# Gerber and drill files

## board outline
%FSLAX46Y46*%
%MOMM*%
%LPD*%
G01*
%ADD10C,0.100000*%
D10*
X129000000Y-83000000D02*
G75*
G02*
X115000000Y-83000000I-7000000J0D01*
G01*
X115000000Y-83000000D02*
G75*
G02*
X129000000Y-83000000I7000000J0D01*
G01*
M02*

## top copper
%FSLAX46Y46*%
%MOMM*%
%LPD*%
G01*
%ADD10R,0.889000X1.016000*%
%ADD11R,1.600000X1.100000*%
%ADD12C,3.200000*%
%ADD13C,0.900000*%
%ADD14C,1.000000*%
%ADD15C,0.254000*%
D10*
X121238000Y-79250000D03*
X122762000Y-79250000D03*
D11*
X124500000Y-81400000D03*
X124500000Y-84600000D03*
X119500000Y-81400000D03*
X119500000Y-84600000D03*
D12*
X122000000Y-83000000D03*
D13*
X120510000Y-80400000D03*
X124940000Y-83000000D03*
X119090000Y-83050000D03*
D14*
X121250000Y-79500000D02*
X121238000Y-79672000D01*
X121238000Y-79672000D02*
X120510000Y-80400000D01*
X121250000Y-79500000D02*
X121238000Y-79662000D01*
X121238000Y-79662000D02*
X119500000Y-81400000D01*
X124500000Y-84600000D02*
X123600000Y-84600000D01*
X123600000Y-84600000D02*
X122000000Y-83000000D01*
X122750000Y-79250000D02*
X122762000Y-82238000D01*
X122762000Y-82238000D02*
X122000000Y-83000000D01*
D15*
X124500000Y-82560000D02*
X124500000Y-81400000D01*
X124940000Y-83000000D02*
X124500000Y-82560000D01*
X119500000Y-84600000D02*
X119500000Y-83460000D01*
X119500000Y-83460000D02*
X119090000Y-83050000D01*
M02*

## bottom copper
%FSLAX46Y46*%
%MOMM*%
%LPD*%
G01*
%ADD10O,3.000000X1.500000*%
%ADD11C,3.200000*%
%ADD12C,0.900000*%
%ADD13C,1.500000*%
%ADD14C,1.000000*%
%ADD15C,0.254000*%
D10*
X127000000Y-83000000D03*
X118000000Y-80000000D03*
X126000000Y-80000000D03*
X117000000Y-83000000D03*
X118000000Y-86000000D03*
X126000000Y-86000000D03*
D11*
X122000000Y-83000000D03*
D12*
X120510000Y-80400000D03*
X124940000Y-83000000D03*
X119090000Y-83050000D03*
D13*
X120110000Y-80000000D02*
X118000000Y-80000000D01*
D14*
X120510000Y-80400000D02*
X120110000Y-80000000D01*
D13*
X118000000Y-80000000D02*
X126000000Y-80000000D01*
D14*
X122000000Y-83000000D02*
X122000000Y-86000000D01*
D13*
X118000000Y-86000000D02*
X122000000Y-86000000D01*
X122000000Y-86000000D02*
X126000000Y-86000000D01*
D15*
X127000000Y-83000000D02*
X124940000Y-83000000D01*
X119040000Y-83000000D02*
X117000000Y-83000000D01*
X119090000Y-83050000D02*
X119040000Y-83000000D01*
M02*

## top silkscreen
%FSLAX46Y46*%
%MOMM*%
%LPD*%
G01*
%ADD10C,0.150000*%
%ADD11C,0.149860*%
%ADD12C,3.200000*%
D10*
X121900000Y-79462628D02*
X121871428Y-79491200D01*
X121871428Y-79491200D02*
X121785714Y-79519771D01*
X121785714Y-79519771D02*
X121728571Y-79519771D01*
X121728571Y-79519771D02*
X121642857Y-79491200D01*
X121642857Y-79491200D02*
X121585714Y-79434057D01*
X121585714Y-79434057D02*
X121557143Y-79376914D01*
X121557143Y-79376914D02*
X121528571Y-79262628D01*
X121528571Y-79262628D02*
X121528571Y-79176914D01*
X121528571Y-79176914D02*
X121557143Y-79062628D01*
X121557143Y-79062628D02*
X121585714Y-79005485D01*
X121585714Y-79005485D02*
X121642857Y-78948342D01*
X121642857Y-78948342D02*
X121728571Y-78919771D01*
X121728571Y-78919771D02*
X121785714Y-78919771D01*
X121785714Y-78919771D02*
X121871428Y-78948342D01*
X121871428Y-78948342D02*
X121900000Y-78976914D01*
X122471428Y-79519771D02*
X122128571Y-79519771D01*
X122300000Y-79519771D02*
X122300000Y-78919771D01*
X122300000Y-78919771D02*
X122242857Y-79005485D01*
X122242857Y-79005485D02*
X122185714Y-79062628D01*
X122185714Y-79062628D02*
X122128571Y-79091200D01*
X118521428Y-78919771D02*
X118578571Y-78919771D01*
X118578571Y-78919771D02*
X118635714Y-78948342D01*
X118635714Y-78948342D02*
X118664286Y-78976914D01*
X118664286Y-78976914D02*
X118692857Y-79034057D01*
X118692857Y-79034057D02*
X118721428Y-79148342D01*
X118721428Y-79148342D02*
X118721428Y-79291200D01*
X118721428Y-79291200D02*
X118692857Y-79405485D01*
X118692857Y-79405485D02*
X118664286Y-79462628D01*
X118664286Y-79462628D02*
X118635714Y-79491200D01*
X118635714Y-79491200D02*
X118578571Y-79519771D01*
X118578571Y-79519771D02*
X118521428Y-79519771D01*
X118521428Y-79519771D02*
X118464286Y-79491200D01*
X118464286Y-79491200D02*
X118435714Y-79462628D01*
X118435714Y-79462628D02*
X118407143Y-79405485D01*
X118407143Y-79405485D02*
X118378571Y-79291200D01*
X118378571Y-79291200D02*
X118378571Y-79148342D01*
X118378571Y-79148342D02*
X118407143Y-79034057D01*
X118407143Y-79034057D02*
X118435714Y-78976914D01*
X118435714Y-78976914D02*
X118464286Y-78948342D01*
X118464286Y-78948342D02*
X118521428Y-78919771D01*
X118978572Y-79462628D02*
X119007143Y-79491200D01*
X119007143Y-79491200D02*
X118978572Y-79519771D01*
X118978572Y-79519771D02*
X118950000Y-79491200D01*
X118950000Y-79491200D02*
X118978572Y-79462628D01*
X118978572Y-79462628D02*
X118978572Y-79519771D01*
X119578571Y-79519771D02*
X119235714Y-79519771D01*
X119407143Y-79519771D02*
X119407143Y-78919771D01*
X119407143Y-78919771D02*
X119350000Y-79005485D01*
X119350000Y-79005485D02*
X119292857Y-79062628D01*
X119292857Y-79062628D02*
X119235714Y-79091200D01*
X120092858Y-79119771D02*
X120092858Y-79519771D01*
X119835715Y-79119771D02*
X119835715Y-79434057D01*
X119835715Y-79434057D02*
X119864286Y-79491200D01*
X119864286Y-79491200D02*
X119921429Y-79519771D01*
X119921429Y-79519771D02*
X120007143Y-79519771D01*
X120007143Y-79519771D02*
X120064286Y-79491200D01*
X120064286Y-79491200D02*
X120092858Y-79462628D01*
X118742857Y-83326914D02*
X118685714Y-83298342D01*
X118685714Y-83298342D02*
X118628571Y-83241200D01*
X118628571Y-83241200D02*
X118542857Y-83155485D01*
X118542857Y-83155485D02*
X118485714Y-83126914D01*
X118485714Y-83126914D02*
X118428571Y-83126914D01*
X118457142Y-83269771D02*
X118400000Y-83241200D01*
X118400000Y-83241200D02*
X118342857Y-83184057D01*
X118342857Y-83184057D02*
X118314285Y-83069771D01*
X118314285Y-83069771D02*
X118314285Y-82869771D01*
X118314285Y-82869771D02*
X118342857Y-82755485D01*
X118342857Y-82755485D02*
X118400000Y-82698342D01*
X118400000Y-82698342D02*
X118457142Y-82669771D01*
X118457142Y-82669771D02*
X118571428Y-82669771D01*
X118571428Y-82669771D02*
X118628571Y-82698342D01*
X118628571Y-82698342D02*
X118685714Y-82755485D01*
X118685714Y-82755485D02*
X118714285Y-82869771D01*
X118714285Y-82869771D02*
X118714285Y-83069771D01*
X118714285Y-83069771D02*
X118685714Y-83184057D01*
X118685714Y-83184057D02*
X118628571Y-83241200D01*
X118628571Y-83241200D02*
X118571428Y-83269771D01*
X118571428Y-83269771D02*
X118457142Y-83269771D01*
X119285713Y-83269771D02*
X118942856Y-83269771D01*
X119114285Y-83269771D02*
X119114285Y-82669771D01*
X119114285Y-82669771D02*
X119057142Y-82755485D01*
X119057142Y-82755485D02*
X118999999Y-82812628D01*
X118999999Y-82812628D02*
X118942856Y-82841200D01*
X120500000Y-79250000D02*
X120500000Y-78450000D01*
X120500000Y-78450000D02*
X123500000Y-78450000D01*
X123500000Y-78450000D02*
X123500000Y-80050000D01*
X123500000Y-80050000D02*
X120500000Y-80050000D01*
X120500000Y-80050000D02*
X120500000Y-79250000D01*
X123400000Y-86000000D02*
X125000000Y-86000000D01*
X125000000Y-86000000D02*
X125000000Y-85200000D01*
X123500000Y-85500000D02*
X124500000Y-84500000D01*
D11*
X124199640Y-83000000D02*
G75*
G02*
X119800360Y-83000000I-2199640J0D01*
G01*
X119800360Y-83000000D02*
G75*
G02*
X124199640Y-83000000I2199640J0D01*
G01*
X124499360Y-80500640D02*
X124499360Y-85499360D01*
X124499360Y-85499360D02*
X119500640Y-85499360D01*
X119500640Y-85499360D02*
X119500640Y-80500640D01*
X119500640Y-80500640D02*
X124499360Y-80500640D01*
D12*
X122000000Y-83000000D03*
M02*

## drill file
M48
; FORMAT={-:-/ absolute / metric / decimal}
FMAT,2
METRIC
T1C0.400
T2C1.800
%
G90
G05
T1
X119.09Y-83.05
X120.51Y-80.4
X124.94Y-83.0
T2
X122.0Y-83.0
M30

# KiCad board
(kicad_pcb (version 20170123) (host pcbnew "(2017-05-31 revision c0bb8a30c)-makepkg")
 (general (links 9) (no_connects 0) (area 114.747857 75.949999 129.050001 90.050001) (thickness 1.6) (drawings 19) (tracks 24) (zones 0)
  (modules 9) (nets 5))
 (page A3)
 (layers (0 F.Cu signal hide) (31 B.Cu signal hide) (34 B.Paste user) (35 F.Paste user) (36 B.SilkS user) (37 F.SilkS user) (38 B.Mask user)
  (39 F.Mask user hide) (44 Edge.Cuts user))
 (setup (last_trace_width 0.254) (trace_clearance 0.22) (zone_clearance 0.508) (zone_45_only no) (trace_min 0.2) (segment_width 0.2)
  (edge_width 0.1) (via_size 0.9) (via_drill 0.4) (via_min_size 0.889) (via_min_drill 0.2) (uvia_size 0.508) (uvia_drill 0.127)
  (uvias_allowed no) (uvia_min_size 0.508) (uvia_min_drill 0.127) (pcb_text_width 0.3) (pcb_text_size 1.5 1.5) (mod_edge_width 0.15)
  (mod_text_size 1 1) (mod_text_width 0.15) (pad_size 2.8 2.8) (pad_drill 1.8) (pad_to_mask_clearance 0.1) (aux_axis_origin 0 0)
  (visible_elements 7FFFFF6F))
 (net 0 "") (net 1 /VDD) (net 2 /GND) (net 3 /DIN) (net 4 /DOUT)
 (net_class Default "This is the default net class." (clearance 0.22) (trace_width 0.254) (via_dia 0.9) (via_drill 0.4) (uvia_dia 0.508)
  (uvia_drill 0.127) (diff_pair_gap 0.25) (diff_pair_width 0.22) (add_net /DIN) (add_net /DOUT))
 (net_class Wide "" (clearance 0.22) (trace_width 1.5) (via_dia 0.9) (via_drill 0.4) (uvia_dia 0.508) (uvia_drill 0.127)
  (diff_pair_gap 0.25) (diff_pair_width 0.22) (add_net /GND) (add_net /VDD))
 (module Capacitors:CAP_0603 (layer F.Cu) (at 122 79.25)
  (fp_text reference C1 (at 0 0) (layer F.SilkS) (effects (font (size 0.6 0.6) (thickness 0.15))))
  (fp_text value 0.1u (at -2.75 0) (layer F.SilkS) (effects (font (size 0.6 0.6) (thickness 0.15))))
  (fp_line (start -1.5 0) (end -1.5 -0.8) (layer F.SilkS) (width 0.15))
  (fp_line (start -1.5 -0.8) (end 1.5 -0.8) (layer F.SilkS) (width 0.15))
  (fp_line (start 1.5 -0.8) (end 1.5 0.8) (layer F.SilkS) (width 0.15))
  (fp_line (start 1.5 0.8) (end -1.5 0.8) (layer F.SilkS) (width 0.15))
  (fp_line (start -1.5 0.8) (end -1.5 0) (layer F.SilkS) (width 0.15))
  (pad 1 smd rect (at -0.762 0) (size 0.889 1.016) (layers F.Cu F.Paste F.Mask) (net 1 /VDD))
  (pad 2 smd rect (at 0.762 0) (size 0.889 1.016) (layers F.Cu F.Paste F.Mask) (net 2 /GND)))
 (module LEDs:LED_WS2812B (layer F.Cu) (at 122 83)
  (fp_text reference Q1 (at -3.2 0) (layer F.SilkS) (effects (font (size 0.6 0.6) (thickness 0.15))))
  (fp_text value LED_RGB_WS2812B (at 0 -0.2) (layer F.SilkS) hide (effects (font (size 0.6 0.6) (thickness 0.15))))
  (fp_line (start 1.4 3) (end 3 3) (layer F.SilkS) (width 0.15))
  (fp_line (start 3 3) (end 3 2.2) (layer F.SilkS) (width 0.15))
  (fp_line (start 1.5 2.5) (end 2.5 1.5) (layer F.SilkS) (width 0.15))
  (fp_circle (center 0 0) (end 0 2.19964) (layer F.SilkS) (width 0.14986))
  (fp_line (start 2.49936 -2.49936) (end 2.49936 2.49936) (layer F.SilkS) (width 0.14986))
  (fp_line (start 2.49936 2.49936) (end -2.49936 2.49936) (layer F.SilkS) (width 0.14986))
  (fp_line (start -2.49936 2.49936) (end -2.49936 -2.49936) (layer F.SilkS) (width 0.14986))
  (fp_line (start -2.49936 -2.49936) (end 2.49936 -2.49936) (layer F.SilkS) (width 0.14986))
  (pad 4 smd rect (at 2.5 -1.6) (size 1.6 1.1) (layers F.Cu F.Paste F.Mask) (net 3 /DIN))
  (pad 3 smd rect (at 2.5 1.6) (size 1.6 1.1) (layers F.Cu F.Paste F.Mask) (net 2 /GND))
  (pad 1 smd rect (at -2.5 -1.6) (size 1.6 1.1) (layers F.Cu F.Paste F.Mask) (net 1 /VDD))
  (pad 2 smd rect (at -2.5 1.6) (size 1.6 1.1) (layers F.Cu F.Paste F.Mask) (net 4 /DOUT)))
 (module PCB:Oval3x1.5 (layer B.Cu) (at 127 83)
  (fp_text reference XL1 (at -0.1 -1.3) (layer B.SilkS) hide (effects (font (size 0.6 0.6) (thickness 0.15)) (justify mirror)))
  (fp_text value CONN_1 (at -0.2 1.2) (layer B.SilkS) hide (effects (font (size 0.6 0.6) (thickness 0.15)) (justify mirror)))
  (pad 1 smd oval (at 0 0) (size 3 1.5) (layers B.Cu B.Paste B.Mask) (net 3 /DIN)))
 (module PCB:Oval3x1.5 (layer B.Cu) (at 118 80)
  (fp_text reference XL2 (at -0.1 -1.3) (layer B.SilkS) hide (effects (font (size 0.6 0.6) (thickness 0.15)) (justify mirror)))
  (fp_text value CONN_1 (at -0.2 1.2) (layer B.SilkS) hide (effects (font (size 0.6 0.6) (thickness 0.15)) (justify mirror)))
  (pad 1 smd oval (at 0 0) (size 3 1.5) (layers B.Cu B.Paste B.Mask) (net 1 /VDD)))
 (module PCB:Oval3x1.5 (layer B.Cu) (at 126 80)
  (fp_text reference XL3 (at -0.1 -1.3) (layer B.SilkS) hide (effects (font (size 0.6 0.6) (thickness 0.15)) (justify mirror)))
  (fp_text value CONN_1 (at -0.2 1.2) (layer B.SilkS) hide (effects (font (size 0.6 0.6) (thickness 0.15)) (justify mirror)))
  (pad 1 smd oval (at 0 0) (size 3 1.5) (layers B.Cu B.Paste B.Mask) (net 1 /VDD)))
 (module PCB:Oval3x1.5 (layer B.Cu) (at 117 83)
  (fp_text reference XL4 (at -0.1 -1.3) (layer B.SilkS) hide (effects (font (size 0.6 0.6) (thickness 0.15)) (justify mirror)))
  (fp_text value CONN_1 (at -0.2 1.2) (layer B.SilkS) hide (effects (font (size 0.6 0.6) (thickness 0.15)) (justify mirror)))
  (pad 1 smd oval (at 0 0) (size 3 1.5) (layers B.Cu B.Paste B.Mask) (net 4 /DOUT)))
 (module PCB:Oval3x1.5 (layer B.Cu) (at 118 86)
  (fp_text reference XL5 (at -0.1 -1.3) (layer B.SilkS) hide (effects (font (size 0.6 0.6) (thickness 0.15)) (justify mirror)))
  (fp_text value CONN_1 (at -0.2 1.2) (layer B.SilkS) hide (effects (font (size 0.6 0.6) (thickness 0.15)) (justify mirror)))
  (pad 1 smd oval (at 0 0) (size 3 1.5) (layers B.Cu B.Paste B.Mask) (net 2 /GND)))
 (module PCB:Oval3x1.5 (layer B.Cu) (at 126 86)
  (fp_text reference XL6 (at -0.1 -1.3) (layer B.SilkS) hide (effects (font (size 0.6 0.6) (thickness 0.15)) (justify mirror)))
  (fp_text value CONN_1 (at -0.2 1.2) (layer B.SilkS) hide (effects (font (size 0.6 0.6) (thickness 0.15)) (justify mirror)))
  (pad 1 smd oval (at 0 0) (size 3 1.5) (layers B.Cu B.Paste B.Mask) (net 2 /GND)))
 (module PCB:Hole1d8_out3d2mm (layer F.Cu) (at 122 83)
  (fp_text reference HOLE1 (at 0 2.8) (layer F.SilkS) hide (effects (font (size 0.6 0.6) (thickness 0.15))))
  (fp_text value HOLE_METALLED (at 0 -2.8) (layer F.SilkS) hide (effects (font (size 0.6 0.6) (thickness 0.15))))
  (pad H thru_hole circle (at 0 0) (size 3.2 3.2) (drill 1.8) (layers *.Cu *.Mask F.SilkS) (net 2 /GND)))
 (gr_circle (center 122 83) (end 129 83) (layer Edge.Cuts) (width 0.1))
 (segment (start 121.25 79.5) (end 121.238 79.672) (width 1) (layer F.Cu) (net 1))
 (segment (start 120.11 80) (end 118 80) (width 1.5) (layer B.Cu) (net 1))
 (segment (start 120.51 80.4) (end 120.11 80) (width 1) (layer B.Cu) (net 1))
 (via (at 120.51 80.4) (size 0.9) (drill 0.4) (layers F.Cu B.Cu) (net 1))
 (segment (start 121.238 79.672) (end 120.51 80.4) (width 1) (layer F.Cu) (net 1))
 (segment (start 121.25 79.5) (end 121.238 79.662) (width 1) (layer F.Cu) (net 1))
 (segment (start 121.238 79.662) (end 119.5 81.4) (width 1) (layer F.Cu) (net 1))
 (segment (start 118 80) (end 126 80) (width 1.5) (layer B.Cu) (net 1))
 (segment (start 122 83) (end 122 86) (width 1) (layer B.Cu) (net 2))
 (segment (start 124.5 84.6) (end 123.6 84.6) (width 1) (layer F.Cu) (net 2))
 (segment (start 123.6 84.6) (end 122 83) (width 1) (layer F.Cu) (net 2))
 (segment (start 122.75 79.25) (end 122.762 82.238) (width 1) (layer F.Cu) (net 2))
 (segment (start 122.762 82.238) (end 122 83) (width 1) (layer F.Cu) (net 2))
 (segment (start 118 86) (end 122 86) (width 1.5) (layer B.Cu) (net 2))
 (segment (start 122 86) (end 126 86) (width 1.5) (layer B.Cu) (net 2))
 (segment (start 127 83) (end 124.94 83) (width 0.254) (layer B.Cu) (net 3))
 (segment (start 124.5 82.56) (end 124.5 81.4) (width 0.254) (layer F.Cu) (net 3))
 (segment (start 124.94 83) (end 124.5 82.56) (width 0.254) (layer F.Cu) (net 3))
 (via (at 124.94 83) (size 0.9) (drill 0.4) (layers F.Cu B.Cu) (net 3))
 (segment (start 119.5 84.6) (end 119.5 83.46) (width 0.254) (layer F.Cu) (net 4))
 (segment (start 119.04 83) (end 117 83) (width 0.254) (layer B.Cu) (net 4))
 (segment (start 119.09 83.05) (end 119.04 83) (width 0.254) (layer B.Cu) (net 4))
 (via (at 119.09 83.05) (size 0.9) (drill 0.4) (layers F.Cu B.Cu) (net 4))
 (segment (start 119.5 83.46) (end 119.09 83.05) (width 0.254) (layer F.Cu) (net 4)))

